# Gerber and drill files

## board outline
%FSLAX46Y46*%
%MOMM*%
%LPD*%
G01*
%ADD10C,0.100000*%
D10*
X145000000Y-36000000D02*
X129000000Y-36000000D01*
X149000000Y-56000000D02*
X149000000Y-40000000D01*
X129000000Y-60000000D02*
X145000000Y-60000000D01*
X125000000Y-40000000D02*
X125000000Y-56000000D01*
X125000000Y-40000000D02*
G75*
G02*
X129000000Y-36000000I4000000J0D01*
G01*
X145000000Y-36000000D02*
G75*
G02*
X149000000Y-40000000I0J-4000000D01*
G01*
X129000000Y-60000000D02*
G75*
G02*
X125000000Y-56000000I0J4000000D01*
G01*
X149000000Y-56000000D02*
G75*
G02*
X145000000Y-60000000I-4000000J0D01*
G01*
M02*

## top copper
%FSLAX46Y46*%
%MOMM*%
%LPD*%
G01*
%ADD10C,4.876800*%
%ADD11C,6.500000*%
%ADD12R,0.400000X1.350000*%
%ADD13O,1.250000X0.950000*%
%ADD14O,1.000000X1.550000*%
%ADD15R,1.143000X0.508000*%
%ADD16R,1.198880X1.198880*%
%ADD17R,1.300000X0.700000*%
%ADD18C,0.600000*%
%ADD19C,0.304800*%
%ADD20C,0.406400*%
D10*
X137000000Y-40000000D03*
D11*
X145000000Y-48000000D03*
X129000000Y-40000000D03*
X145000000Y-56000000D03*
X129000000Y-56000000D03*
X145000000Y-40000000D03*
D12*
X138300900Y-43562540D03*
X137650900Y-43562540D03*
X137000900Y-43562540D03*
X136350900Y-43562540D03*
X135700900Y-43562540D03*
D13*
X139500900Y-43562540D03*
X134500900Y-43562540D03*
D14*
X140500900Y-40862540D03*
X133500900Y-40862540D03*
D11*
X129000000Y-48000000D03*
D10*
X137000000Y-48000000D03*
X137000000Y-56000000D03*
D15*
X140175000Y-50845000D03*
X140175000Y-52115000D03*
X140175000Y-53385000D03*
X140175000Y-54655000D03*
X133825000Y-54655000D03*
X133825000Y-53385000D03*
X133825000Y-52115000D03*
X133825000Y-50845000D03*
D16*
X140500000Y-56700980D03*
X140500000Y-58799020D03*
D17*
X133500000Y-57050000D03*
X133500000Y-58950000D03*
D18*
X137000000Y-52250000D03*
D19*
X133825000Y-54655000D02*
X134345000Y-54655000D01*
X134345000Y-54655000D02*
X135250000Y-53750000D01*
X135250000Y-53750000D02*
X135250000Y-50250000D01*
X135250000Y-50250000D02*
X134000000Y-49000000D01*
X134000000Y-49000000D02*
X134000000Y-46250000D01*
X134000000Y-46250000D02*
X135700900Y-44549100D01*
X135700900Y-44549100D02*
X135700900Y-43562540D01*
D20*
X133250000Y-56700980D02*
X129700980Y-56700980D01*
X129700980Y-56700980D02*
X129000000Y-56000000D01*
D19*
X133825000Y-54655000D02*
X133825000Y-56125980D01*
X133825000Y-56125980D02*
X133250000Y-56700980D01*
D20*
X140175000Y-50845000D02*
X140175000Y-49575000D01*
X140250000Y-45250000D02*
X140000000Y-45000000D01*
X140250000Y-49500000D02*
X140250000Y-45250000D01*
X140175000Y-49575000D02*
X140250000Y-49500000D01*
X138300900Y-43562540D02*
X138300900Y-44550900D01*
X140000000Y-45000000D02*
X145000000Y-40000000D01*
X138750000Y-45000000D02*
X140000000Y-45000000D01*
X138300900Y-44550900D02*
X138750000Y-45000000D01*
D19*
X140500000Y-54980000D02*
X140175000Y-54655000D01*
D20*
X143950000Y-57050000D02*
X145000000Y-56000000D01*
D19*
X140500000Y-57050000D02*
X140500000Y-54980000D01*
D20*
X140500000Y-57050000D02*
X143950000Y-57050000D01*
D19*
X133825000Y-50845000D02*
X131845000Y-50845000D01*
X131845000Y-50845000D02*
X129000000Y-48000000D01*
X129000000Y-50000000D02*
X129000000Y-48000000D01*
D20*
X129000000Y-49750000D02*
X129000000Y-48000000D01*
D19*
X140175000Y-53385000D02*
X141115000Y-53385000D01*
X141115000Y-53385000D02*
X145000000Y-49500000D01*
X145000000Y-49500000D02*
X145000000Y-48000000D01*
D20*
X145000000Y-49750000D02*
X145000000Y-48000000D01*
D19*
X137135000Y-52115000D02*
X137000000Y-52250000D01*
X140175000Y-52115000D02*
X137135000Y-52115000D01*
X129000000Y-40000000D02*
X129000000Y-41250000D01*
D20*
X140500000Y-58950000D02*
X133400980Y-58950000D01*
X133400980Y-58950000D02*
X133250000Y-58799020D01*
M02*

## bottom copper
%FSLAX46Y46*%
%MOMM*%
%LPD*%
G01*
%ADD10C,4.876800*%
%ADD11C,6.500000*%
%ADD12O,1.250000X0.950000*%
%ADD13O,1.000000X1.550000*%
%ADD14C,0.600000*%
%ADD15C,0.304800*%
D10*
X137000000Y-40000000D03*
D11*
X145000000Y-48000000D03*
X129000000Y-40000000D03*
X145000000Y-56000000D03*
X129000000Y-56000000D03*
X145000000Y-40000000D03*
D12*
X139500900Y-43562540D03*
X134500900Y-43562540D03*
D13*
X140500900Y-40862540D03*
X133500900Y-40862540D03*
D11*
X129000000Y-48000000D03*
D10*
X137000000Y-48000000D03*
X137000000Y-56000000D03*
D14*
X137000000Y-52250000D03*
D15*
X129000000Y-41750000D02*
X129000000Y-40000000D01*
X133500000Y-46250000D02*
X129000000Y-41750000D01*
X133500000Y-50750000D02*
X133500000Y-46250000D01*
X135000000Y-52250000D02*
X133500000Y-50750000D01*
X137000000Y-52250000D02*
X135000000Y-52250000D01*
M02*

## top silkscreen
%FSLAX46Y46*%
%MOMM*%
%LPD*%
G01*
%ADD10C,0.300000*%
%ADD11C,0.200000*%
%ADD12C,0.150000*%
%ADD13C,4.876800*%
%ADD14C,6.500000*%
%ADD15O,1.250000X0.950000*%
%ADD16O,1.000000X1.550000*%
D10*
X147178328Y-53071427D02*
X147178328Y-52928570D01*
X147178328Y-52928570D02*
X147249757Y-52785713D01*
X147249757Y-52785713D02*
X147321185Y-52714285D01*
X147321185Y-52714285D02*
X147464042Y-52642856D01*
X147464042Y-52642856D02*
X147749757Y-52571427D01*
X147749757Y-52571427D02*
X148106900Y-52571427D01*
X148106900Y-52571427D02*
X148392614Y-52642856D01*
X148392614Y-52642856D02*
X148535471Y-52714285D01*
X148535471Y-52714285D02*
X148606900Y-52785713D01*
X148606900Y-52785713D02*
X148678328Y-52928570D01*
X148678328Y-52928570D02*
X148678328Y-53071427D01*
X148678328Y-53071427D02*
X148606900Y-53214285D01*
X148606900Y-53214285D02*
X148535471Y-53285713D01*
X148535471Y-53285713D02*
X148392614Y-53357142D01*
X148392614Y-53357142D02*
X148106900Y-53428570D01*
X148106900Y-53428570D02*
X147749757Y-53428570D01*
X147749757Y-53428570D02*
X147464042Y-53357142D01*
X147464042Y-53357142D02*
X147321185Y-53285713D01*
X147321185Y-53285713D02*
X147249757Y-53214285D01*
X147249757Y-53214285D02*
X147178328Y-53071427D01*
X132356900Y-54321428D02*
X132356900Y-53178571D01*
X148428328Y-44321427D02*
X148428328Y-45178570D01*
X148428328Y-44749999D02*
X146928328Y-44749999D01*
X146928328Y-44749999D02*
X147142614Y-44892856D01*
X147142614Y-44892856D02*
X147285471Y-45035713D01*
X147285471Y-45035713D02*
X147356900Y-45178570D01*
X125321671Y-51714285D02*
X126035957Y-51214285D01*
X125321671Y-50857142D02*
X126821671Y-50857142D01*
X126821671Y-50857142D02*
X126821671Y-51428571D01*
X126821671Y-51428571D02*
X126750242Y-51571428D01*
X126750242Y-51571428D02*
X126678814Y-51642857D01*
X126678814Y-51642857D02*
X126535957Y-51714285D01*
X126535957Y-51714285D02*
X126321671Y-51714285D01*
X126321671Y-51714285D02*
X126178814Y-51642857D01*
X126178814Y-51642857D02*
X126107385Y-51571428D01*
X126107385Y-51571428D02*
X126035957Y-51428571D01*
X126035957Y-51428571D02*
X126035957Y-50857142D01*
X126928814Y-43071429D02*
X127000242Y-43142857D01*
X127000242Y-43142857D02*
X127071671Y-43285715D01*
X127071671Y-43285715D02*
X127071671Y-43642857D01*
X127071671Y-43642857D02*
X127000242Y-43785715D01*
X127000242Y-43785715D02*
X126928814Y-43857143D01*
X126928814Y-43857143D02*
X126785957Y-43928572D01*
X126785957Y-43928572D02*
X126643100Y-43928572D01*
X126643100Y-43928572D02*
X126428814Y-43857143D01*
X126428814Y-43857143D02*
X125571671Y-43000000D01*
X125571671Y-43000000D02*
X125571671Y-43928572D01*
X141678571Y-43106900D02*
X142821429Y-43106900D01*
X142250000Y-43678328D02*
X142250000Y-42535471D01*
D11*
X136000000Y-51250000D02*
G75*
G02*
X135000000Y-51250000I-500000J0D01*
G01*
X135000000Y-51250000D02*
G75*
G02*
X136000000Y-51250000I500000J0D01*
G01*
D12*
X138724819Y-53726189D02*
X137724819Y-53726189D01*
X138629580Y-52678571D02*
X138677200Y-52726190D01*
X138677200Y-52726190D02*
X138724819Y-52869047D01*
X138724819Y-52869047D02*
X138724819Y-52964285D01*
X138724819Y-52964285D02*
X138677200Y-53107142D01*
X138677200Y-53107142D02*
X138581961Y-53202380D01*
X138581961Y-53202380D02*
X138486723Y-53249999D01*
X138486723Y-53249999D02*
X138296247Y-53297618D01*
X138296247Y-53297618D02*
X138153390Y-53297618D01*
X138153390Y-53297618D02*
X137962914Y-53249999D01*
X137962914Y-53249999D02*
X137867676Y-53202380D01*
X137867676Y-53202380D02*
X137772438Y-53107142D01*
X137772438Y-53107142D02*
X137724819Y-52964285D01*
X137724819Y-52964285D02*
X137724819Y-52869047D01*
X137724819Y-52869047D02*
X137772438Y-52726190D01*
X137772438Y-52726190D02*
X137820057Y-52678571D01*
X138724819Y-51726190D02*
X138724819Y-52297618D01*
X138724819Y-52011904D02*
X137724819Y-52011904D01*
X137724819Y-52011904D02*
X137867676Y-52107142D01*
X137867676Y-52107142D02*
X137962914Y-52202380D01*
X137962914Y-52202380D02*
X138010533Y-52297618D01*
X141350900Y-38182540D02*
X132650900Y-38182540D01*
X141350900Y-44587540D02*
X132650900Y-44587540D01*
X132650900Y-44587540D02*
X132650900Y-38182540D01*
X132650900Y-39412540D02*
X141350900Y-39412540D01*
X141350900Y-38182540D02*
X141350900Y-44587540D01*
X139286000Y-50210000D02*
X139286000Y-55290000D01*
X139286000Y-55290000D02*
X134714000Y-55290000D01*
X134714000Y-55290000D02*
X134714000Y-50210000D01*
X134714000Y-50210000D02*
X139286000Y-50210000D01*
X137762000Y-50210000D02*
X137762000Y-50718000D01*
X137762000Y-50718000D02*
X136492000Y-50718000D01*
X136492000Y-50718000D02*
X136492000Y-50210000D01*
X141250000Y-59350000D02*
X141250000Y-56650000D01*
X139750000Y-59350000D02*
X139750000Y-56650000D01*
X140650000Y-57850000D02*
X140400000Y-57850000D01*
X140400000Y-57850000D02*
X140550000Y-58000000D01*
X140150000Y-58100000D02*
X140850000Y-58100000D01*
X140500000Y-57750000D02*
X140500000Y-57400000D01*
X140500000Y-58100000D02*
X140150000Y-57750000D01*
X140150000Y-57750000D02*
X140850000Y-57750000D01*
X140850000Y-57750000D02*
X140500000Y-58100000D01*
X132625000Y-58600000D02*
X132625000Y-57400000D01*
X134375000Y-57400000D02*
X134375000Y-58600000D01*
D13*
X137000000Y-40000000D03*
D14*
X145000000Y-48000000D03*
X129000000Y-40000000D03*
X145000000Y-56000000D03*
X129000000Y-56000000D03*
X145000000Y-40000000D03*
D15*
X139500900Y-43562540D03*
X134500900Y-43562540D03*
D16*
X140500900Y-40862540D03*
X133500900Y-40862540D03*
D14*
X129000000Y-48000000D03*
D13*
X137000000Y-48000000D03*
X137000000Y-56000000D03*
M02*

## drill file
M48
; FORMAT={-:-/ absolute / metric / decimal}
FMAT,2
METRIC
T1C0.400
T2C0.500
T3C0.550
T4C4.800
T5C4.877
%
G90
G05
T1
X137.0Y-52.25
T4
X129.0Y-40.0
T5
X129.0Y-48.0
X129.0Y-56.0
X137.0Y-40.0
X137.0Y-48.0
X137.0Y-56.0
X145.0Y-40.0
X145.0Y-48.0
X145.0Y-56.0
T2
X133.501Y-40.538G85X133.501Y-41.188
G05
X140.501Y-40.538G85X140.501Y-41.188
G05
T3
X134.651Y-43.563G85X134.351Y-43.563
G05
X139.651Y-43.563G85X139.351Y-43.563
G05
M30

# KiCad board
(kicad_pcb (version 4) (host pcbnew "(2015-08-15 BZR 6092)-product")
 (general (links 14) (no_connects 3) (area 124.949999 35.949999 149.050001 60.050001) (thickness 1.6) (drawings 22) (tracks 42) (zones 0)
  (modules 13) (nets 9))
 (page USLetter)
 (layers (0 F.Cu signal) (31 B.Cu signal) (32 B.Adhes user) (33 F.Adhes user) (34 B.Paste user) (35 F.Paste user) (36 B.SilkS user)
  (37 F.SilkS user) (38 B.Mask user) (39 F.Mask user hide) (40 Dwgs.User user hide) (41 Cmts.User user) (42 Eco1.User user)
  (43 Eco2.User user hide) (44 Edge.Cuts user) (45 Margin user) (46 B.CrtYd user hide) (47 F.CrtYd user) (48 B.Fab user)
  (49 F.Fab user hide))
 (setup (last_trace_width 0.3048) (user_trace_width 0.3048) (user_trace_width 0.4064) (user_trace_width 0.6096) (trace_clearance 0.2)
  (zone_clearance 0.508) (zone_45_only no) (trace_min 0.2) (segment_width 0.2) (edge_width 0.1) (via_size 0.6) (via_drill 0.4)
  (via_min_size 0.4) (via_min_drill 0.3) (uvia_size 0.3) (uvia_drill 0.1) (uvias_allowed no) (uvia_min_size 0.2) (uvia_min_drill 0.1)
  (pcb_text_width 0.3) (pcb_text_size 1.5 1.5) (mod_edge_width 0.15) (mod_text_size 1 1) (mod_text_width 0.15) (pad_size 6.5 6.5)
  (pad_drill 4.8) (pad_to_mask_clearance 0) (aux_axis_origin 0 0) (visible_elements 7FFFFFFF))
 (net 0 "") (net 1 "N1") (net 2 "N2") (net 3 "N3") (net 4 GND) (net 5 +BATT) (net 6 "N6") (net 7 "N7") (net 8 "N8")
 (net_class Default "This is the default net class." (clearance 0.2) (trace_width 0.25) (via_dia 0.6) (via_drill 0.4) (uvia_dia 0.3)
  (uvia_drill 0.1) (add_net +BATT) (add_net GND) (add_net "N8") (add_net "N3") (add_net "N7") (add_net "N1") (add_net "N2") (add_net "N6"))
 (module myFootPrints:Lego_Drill (layer F.Cu) (at 137 40)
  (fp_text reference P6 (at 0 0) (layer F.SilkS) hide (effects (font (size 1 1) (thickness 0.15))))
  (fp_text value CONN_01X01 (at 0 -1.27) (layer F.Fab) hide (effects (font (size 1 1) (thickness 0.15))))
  (pad 1 thru_hole circle (at 0 0) (size 4.8768 4.8768) (drill 4.8768) (layers *.Cu *.Mask F.SilkS)))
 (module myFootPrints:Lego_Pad (layer F.Cu) (at 145 48 180)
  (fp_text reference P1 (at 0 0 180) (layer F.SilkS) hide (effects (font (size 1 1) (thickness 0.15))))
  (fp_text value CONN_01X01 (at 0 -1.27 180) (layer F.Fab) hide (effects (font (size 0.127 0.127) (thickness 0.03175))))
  (pad 1 thru_hole circle (at 0 0 180) (size 6.5 6.5) (drill 4.8768) (layers *.Cu *.Mask F.SilkS) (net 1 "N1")))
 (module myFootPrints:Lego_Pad (layer F.Cu) (at 129 40)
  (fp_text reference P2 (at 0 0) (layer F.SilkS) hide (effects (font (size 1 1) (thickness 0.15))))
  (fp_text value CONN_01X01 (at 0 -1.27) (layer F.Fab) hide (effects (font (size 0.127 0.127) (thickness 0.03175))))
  (pad 1 thru_hole circle (at 0 0) (size 6.5 6.5) (drill 4.8) (layers *.Cu *.Mask F.SilkS) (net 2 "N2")))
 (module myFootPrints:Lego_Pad (layer F.Cu) (at 145 56)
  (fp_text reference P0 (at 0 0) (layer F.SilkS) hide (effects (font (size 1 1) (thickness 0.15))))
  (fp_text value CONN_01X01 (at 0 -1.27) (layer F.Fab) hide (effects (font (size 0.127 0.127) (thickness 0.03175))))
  (pad 1 thru_hole circle (at 0 0) (size 6.5 6.5) (drill 4.8768) (layers *.Cu *.Mask F.SilkS) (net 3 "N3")))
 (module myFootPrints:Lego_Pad (layer F.Cu) (at 129 56)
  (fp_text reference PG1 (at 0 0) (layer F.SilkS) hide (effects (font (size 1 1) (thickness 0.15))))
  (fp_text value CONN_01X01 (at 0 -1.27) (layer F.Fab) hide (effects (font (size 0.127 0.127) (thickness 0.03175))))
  (pad 1 thru_hole circle (at 0 0) (size 6.5 6.5) (drill 4.8768) (layers *.Cu *.Mask F.SilkS) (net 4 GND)))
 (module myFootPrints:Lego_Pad (layer F.Cu) (at 145 40)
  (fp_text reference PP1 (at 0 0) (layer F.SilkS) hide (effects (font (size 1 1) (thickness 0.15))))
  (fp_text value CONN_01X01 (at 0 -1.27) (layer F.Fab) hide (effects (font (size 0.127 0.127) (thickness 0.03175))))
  (pad 1 thru_hole circle (at 0 0) (size 6.5 6.5) (drill 4.8768) (layers *.Cu *.Mask F.SilkS) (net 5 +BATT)))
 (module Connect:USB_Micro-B (layer F.Cu) (at 137 42 180)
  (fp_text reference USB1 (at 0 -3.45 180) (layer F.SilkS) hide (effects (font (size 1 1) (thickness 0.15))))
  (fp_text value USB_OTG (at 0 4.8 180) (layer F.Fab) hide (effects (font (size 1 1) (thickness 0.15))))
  (fp_line (start -4.3509 3.81746) (end 4.3491 3.81746) (layer F.SilkS) (width 0.15))
  (fp_line (start -4.3509 -2.58754) (end 4.3491 -2.58754) (layer F.SilkS) (width 0.15))
  (fp_line (start 4.3491 -2.58754) (end 4.3491 3.81746) (layer F.SilkS) (width 0.15))
  (fp_line (start 4.3491 2.58746) (end -4.3509 2.58746) (layer F.SilkS) (width 0.15))
  (fp_line (start -4.3509 3.81746) (end -4.3509 -2.58754) (layer F.SilkS) (width 0.15))
  (pad 1 smd rect (at -1.3009 -1.56254 270) (size 1.35 0.4) (layers F.Cu F.Paste F.Mask) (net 5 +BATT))
  (pad 2 smd rect (at -0.6509 -1.56254 270) (size 1.35 0.4) (layers F.Cu F.Paste F.Mask))
  (pad 3 smd rect (at -0.0009 -1.56254 270) (size 1.35 0.4) (layers F.Cu F.Paste F.Mask))
  (pad 4 smd rect (at 0.6491 -1.56254 270) (size 1.35 0.4) (layers F.Cu F.Paste F.Mask))
  (pad 5 smd rect (at 1.2991 -1.56254 270) (size 1.35 0.4) (layers F.Cu F.Paste F.Mask) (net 4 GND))
  (pad 6 thru_hole oval (at -2.5009 -1.56254 270) (size 0.95 1.25) (drill oval 0.55 0.85) (layers *.Cu *.Mask F.SilkS) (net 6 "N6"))
  (pad 6 thru_hole oval (at 2.4991 -1.56254 270) (size 0.95 1.25) (drill oval 0.55 0.85) (layers *.Cu *.Mask F.SilkS) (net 6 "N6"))
  (pad 6 thru_hole oval (at -3.5009 1.13746 270) (size 1.55 1) (drill oval 1.15 0.5) (layers *.Cu *.Mask F.SilkS) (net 6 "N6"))
  (pad 6 thru_hole oval (at 3.4991 1.13746 270) (size 1.55 1) (drill oval 1.15 0.5) (layers *.Cu *.Mask F.SilkS) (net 6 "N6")))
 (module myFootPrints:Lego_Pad (layer F.Cu) (at 129 48)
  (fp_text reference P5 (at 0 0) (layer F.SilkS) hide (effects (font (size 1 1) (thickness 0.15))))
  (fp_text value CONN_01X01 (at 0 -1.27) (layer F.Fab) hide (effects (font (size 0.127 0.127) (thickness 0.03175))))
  (pad 1 thru_hole circle (at 0 0) (size 6.5 6.5) (drill 4.8768) (layers *.Cu *.Mask F.SilkS) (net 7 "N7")))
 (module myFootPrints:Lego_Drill (layer F.Cu) (at 137 48)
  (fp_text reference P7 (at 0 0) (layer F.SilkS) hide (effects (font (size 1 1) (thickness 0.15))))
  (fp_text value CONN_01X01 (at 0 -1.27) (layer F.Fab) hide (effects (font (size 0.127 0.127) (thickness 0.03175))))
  (pad 1 thru_hole circle (at 0 0) (size 4.8768 4.8768) (drill 4.8768) (layers *.Cu *.Mask F.SilkS)))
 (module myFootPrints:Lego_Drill (layer F.Cu) (at 137 56)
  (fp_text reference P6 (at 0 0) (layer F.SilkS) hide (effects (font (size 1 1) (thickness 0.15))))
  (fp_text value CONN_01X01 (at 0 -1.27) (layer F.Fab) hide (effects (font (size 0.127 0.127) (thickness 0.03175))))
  (pad 1 thru_hole circle (at 0 0) (size 4.8768 4.8768) (drill 4.8768) (layers *.Cu *.Mask F.SilkS)))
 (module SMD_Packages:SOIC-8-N (layer F.Cu) (at 137 52.75 270)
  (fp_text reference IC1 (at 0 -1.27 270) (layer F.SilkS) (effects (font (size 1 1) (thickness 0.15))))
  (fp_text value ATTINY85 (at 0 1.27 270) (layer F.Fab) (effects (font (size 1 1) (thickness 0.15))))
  (fp_line (start -2.54 -2.286) (end 2.54 -2.286) (layer F.SilkS) (width 0.15))
  (fp_line (start 2.54 -2.286) (end 2.54 2.286) (layer F.SilkS) (width 0.15))
  (fp_line (start 2.54 2.286) (end -2.54 2.286) (layer F.SilkS) (width 0.15))
  (fp_line (start -2.54 2.286) (end -2.54 -2.286) (layer F.SilkS) (width 0.15))
  (fp_line (start -2.54 -0.762) (end -2.032 -0.762) (layer F.SilkS) (width 0.15))
  (fp_line (start -2.032 -0.762) (end -2.032 0.508) (layer F.SilkS) (width 0.15))
  (fp_line (start -2.032 0.508) (end -2.54 0.508) (layer F.SilkS) (width 0.15))
  (pad 8 smd rect (at -1.905 -3.175 270) (size 0.508 1.143) (layers F.Cu F.Paste F.Mask) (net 5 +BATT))
  (pad 7 smd rect (at -0.635 -3.175 270) (size 0.508 1.143) (layers F.Cu F.Paste F.Mask) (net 2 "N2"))
  (pad 6 smd rect (at 0.635 -3.175 270) (size 0.508 1.143) (layers F.Cu F.Paste F.Mask) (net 1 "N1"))
  (pad 5 smd rect (at 1.905 -3.175 270) (size 0.508 1.143) (layers F.Cu F.Paste F.Mask) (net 3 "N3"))
  (pad 4 smd rect (at 1.905 3.175 270) (size 0.508 1.143) (layers F.Cu F.Paste F.Mask) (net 4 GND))
  (pad 3 smd rect (at 0.635 3.175 270) (size 0.508 1.143) (layers F.Cu F.Paste F.Mask))
  (pad 2 smd rect (at -0.635 3.175 270) (size 0.508 1.143) (layers F.Cu F.Paste F.Mask))
  (pad 1 smd rect (at -1.905 3.175 270) (size 0.508 1.143) (layers F.Cu F.Paste F.Mask) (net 7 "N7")))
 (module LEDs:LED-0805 (layer F.Cu) (at 140.5 57.75 90)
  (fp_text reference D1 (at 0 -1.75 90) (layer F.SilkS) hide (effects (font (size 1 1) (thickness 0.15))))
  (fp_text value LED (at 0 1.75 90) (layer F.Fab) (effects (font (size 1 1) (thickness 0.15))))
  (fp_line (start -1.6 0.75) (end 1.1 0.75) (layer F.SilkS) (width 0.15))
  (fp_line (start -1.6 -0.75) (end 1.1 -0.75) (layer F.SilkS) (width 0.15))
  (fp_line (start -0.1 0.15) (end -0.1 -0.1) (layer F.SilkS) (width 0.15))
  (fp_line (start -0.1 -0.1) (end -0.25 0.05) (layer F.SilkS) (width 0.15))
  (fp_line (start -0.35 -0.35) (end -0.35 0.35) (layer F.SilkS) (width 0.15))
  (fp_line (start 0 0) (end 0.35 0) (layer F.SilkS) (width 0.15))
  (fp_line (start -0.35 0) (end 0 -0.35) (layer F.SilkS) (width 0.15))
  (fp_line (start 0 -0.35) (end 0 0.35) (layer F.SilkS) (width 0.15))
  (fp_line (start 0 0.35) (end -0.35 0) (layer F.SilkS) (width 0.15))
  (pad 2 smd rect (at 1.04902 0 270) (size 1.19888 1.19888) (layers F.Cu F.Paste F.Mask) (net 3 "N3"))
  (pad 1 smd rect (at -1.04902 0 270) (size 1.19888 1.19888) (layers F.Cu F.Paste F.Mask) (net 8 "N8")))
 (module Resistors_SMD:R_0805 (layer F.Cu) (at 133.5 58 270)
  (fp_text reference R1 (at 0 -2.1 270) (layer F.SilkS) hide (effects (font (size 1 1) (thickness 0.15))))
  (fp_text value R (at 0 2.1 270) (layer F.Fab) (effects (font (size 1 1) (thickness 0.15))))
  (fp_line (start 0.6 0.875) (end -0.6 0.875) (layer F.SilkS) (width 0.15))
  (fp_line (start -0.6 -0.875) (end 0.6 -0.875) (layer F.SilkS) (width 0.15))
  (pad 1 smd rect (at -0.95 0 270) (size 0.7 1.3) (layers F.Cu F.Paste F.Mask) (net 4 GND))
  (pad 2 smd rect (at 0.95 0 270) (size 0.7 1.3) (layers F.Cu F.Paste F.Mask) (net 8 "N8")))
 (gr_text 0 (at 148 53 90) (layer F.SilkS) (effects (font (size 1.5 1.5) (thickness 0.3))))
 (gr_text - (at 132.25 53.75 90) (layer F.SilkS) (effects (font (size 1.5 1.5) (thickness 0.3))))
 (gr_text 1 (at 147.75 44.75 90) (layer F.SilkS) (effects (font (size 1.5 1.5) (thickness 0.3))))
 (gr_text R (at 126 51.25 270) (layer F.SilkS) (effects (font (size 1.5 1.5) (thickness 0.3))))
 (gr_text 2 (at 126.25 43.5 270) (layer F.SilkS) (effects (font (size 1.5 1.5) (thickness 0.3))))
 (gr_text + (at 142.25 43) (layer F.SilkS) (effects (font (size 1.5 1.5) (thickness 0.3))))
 (gr_circle (center 135.5 51.25) (end 135.5 50.75) (layer F.SilkS) (width 0.2))
 (gr_line (start 145 36) (end 129 36) (angle 90) (layer Edge.Cuts) (width 0.1))
 (gr_line (start 149 56) (end 149 40) (angle 90) (layer Edge.Cuts) (width 0.1))
 (gr_line (start 129 60) (end 145 60) (angle 90) (layer Edge.Cuts) (width 0.1))
 (gr_line (start 125 40) (end 125 56) (angle 90) (layer Edge.Cuts) (width 0.1))
 (gr_arc (start 129 40) (end 125 40) (angle 90) (layer Edge.Cuts) (width 0.1))
 (gr_arc (start 145 40) (end 145 36) (angle 90) (layer Edge.Cuts) (width 0.1))
 (gr_arc (start 129 56) (end 129 60) (angle 90) (layer Edge.Cuts) (width 0.1))
 (gr_arc (start 145 56) (end 149 56) (angle 90) (layer Edge.Cuts) (width 0.1))
 (segment (start 133.825 54.655) (end 134.345 54.655) (width 0.3048) (layer F.Cu) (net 4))
 (segment (start 134.345 54.655) (end 135.25 53.75) (width 0.3048) (layer F.Cu) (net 4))
 (segment (start 135.25 53.75) (end 135.25 50.25) (width 0.3048) (layer F.Cu) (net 4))
 (segment (start 135.25 50.25) (end 134 49) (width 0.3048) (layer F.Cu) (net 4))
 (segment (start 134 49) (end 134 46.25) (width 0.3048) (layer F.Cu) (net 4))
 (segment (start 134 46.25) (end 135.7009 44.5491) (width 0.3048) (layer F.Cu) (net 4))
 (segment (start 135.7009 44.5491) (end 135.7009 43.56254) (width 0.3048) (layer F.Cu) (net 4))
 (segment (start 133.25 56.70098) (end 129.70098 56.70098) (width 0.4064) (layer F.Cu) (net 4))
 (segment (start 129.70098 56.70098) (end 129 56) (width 0.4064) (layer F.Cu) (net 4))
 (segment (start 133.825 54.655) (end 133.825 56.12598) (width 0.3048) (layer F.Cu) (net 4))
 (segment (start 133.825 56.12598) (end 133.25 56.70098) (width 0.3048) (layer F.Cu) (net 4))
 (segment (start 140.175 50.845) (end 140.175 49.575) (width 0.4064) (layer F.Cu) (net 5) (status 10))
 (segment (start 140.25 45.25) (end 140 45) (width 0.4064) (layer F.Cu) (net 5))
 (segment (start 140.25 49.5) (end 140.25 45.25) (width 0.4064) (layer F.Cu) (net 5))
 (segment (start 140.175 49.575) (end 140.25 49.5) (width 0.4064) (layer F.Cu) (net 5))
 (segment (start 138.3009 43.56254) (end 138.3009 44.5509) (width 0.4064) (layer F.Cu) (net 5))
 (segment (start 140 45) (end 145 40) (width 0.4064) (layer F.Cu) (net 5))
 (segment (start 138.75 45) (end 140 45) (width 0.4064) (layer F.Cu) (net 5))
 (segment (start 138.3009 44.5509) (end 138.75 45) (width 0.4064) (layer F.Cu) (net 5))
 (segment (start 140.5 54.98) (end 140.175 54.655) (width 0.3048) (layer F.Cu) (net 3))
 (segment (start 143.95 57.05) (end 145 56) (width 0.4064) (layer F.Cu) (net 3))
 (segment (start 140.5 57.05) (end 140.5 54.98) (width 0.3048) (layer F.Cu) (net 3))
 (segment (start 140.5 57.05) (end 143.95 57.05) (width 0.4064) (layer F.Cu) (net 3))
 (segment (start 133.825 50.845) (end 131.845 50.845) (width 0.3048) (layer F.Cu) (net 7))
 (segment (start 131.845 50.845) (end 129 48) (width 0.3048) (layer F.Cu) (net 7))
 (segment (start 129 50) (end 129 48) (width 0.3048) (layer F.Cu) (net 7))
 (segment (start 129 49.75) (end 129 48) (width 0.4064) (layer F.Cu) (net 7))
 (segment (start 140.175 53.385) (end 141.115 53.385) (width 0.3048) (layer F.Cu) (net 1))
 (segment (start 141.115 53.385) (end 145 49.5) (width 0.3048) (layer F.Cu) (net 1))
 (segment (start 145 49.5) (end 145 48) (width 0.3048) (layer F.Cu) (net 1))
 (segment (start 145 49.75) (end 145 48) (width 0.4064) (layer F.Cu) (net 1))
 (segment (start 129 41.75) (end 129 40) (width 0.3048) (layer B.Cu) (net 2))
 (segment (start 133.5 46.25) (end 129 41.75) (width 0.3048) (layer B.Cu) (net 2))
 (segment (start 133.5 50.75) (end 133.5 46.25) (width 0.3048) (layer B.Cu) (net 2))
 (segment (start 135 52.25) (end 133.5 50.75) (width 0.3048) (layer B.Cu) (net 2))
 (segment (start 137 52.25) (end 135 52.25) (width 0.3048) (layer B.Cu) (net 2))
 (via (at 137 52.25) (size 0.6) (drill 0.4) (layers F.Cu B.Cu) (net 2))
 (segment (start 137.135 52.115) (end 137 52.25) (width 0.3048) (layer F.Cu) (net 2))
 (segment (start 140.175 52.115) (end 137.135 52.115) (width 0.3048) (layer F.Cu) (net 2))
 (segment (start 129 40) (end 129 41.25) (width 0.3048) (layer F.Cu) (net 2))
 (segment (start 140.5 58.95) (end 133.40098 58.95) (width 0.4064) (layer F.Cu) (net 8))
 (segment (start 133.40098 58.95) (end 133.25 58.79902) (width 0.4064) (layer F.Cu) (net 8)))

